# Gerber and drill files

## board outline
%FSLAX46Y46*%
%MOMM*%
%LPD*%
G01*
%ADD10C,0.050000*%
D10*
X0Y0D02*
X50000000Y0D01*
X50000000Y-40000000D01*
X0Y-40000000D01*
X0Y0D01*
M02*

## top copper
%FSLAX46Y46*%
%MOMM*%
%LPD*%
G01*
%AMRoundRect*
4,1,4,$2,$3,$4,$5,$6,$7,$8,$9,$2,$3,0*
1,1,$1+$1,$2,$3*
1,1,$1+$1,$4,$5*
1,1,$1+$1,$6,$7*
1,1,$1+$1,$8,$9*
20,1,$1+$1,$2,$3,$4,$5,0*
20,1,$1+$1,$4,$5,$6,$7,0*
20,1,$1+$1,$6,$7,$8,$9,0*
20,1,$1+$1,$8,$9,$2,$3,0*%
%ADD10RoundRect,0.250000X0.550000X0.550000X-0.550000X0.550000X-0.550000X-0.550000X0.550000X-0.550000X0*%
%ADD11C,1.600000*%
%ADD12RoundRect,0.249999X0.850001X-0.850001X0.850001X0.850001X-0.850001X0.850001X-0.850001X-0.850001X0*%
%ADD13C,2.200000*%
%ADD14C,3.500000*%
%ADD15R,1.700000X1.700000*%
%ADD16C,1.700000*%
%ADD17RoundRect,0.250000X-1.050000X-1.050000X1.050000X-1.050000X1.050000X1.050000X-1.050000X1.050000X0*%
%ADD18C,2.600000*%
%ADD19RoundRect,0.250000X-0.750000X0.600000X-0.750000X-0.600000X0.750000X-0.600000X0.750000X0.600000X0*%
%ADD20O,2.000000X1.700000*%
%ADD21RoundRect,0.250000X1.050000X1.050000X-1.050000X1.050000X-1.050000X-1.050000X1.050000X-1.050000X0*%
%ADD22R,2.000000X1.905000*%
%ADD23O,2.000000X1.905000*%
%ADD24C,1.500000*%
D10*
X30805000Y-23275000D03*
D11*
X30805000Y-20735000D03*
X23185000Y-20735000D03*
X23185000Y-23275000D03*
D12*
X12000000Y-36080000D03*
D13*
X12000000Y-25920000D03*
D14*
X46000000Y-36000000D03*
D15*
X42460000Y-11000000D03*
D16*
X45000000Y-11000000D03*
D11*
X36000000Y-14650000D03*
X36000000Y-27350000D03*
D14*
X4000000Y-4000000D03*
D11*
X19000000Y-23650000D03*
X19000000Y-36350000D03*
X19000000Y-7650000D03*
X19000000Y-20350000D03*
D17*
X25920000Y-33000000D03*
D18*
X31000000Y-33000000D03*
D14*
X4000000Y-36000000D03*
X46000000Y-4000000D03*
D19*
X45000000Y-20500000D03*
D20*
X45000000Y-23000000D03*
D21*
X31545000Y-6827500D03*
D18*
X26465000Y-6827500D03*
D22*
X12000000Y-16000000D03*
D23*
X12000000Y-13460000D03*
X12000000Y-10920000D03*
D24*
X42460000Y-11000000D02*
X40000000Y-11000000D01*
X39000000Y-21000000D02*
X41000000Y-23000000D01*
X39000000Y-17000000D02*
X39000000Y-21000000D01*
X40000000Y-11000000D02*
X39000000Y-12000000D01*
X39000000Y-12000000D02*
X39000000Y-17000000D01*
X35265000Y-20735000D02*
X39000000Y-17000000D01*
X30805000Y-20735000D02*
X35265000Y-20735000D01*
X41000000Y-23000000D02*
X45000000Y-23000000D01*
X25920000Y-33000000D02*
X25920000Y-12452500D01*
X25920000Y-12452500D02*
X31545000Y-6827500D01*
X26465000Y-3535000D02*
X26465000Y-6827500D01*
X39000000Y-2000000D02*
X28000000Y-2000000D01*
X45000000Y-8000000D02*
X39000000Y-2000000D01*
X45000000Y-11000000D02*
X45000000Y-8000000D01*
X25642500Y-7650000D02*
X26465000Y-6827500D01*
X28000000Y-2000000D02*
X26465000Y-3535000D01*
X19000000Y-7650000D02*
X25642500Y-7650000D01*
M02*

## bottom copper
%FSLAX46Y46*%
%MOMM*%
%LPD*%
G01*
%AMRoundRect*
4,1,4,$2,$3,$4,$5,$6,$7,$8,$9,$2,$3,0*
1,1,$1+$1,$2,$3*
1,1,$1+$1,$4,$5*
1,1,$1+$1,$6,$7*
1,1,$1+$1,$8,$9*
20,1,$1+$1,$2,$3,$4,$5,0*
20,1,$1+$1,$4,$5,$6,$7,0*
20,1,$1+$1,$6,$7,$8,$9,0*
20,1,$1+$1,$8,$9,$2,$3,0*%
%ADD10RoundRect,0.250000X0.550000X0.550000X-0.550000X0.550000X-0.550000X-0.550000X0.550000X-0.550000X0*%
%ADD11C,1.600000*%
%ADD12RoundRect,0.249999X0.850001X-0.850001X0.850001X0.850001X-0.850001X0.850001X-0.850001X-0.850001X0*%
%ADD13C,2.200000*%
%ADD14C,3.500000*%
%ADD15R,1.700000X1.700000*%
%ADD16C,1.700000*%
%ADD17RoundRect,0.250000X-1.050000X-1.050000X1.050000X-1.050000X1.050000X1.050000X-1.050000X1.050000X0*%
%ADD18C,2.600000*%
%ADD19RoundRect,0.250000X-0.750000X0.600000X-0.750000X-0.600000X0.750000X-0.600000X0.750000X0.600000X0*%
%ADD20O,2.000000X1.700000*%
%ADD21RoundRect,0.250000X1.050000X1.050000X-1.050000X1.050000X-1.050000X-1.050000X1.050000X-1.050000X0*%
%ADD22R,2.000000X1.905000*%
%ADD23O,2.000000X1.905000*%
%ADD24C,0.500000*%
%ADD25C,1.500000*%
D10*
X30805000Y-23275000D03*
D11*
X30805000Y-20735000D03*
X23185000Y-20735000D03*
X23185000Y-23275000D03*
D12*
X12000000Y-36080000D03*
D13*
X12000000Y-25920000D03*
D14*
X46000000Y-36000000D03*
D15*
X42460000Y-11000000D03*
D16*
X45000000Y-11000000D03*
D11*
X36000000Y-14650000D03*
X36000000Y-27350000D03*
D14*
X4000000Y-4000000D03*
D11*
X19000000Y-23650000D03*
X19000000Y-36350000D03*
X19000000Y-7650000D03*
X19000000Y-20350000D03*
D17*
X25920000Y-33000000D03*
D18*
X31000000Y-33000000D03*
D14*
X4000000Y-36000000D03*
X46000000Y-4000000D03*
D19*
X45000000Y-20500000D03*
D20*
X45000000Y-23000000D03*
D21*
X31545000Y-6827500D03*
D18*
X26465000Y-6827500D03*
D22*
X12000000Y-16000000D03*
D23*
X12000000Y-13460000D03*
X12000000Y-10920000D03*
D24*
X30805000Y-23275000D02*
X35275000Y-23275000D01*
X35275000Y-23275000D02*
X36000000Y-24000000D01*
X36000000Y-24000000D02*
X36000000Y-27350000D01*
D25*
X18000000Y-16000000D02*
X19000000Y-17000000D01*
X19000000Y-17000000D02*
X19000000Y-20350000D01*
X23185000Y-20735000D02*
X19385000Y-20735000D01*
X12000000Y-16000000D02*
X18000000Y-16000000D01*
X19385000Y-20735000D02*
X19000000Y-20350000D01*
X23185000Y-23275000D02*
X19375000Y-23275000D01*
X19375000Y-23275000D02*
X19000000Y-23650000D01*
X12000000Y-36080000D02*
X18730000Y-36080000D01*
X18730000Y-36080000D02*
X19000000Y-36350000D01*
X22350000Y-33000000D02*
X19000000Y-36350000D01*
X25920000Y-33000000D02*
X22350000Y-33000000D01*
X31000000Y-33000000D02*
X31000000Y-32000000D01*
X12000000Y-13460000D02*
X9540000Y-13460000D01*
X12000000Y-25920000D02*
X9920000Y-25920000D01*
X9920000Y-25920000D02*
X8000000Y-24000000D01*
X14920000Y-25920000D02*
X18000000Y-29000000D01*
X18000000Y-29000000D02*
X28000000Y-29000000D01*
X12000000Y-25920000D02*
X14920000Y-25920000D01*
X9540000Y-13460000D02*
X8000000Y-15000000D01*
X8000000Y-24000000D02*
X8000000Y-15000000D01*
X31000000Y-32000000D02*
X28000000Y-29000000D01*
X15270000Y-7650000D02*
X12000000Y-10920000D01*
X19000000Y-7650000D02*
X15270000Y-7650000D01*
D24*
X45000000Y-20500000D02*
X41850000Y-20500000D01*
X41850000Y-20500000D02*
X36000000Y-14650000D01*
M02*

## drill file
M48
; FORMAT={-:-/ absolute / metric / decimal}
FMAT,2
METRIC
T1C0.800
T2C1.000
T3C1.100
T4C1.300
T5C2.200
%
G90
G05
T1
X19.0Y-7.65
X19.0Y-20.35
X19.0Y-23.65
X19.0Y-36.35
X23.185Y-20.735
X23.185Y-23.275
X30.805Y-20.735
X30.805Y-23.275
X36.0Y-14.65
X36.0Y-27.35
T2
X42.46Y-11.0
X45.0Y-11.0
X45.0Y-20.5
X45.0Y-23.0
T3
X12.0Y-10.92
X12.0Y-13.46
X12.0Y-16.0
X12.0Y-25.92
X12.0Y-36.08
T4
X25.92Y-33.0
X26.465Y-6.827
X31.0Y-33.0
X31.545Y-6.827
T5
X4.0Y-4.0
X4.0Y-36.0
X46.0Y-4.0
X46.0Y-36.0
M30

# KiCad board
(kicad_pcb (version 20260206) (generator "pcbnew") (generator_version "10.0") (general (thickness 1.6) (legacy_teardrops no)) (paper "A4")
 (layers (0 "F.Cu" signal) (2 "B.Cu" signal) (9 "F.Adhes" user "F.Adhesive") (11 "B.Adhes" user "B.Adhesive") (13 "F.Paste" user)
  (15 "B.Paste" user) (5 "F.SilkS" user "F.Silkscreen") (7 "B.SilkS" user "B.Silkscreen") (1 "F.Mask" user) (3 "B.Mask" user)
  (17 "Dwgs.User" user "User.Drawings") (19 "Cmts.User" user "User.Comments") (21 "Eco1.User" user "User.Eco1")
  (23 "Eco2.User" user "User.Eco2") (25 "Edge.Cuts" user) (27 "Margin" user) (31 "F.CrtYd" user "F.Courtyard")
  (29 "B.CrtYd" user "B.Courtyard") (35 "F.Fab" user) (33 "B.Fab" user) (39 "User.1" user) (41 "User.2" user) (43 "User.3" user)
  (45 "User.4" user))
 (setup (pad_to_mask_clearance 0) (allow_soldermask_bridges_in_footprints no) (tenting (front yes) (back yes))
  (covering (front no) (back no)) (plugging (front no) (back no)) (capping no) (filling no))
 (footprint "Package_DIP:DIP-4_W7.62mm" (layer "F.Cu") (at 30.805 23.275 180)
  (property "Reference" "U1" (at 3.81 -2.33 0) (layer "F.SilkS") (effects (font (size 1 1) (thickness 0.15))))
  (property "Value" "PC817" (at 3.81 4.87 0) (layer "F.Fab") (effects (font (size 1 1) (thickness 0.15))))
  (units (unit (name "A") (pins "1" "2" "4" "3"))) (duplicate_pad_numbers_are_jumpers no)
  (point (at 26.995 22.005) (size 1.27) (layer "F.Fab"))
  (pad "1" thru_hole roundrect (at 0 0 180) (size 1.6 1.6) (drill 0.8) (layers "*.Cu" "*.Mask") (remove_unused_layers no)
   (roundrect_rratio 0.15625) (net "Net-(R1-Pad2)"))
  (pad "2" thru_hole circle (at 0 2.54 180) (size 1.6 1.6) (drill 0.8) (layers "*.Cu" "*.Mask") (remove_unused_layers no) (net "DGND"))
  (pad "3" thru_hole circle (at 7.62 2.54 180) (size 1.6 1.6) (drill 0.8) (layers "*.Cu" "*.Mask") (remove_unused_layers no)
   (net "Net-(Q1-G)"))
  (pad "4" thru_hole circle (at 7.62 0 180) (size 1.6 1.6) (drill 0.8) (layers "*.Cu" "*.Mask") (remove_unused_layers no)
   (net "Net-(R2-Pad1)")))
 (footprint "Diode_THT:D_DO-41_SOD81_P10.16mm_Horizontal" (layer "F.Cu") (at 12 36.08 90)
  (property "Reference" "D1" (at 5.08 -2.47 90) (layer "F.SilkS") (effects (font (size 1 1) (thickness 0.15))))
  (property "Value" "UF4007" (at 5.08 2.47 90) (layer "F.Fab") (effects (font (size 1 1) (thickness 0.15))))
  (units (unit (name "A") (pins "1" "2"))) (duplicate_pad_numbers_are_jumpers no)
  (pad "1" thru_hole roundrect (at 0 0 90) (size 2.2 2.2) (drill 1.1) (layers "*.Cu" "*.Mask") (remove_unused_layers no)
   (roundrect_rratio 0.113636) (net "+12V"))
  (pad "2" thru_hole circle (at 10.16 0 90) (size 2.2 2.2) (drill 1.1) (layers "*.Cu" "*.Mask") (remove_unused_layers no) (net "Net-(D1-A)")))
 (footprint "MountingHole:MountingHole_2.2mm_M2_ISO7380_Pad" (layer "F.Cu") (at 46 36)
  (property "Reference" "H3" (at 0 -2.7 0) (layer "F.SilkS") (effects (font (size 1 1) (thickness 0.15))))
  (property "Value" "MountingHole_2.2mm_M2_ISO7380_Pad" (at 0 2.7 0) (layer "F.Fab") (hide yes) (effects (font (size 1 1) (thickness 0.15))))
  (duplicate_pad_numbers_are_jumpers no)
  (pad "3" thru_hole circle (at 0 0) (size 3.5 3.5) (drill 2.2) (layers "*.Cu" "*.Mask") (remove_unused_layers no) (zone_connect 2)))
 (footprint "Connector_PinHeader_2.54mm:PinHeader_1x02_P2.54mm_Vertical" (layer "F.Cu") (at 42.46 11 90)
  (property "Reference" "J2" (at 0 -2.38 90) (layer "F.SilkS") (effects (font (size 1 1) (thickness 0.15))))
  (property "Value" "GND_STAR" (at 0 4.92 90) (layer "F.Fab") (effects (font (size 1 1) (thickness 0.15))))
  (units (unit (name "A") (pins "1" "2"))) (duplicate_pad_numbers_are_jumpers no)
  (pad "1" thru_hole rect (at 0 0 90) (size 1.7 1.7) (drill 1) (layers "*.Cu" "*.Mask") (remove_unused_layers no) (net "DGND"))
  (pad "2" thru_hole circle (at 0 2.54 90) (size 1.7 1.7) (drill 1) (layers "*.Cu" "*.Mask") (remove_unused_layers no) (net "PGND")))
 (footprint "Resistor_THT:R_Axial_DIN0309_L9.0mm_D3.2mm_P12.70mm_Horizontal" (layer "F.Cu") (at 36 14.65 -90)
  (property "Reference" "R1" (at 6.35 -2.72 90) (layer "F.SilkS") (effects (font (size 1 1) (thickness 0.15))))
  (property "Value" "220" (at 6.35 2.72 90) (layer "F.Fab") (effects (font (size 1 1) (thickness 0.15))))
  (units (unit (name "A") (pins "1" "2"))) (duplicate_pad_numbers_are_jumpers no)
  (pad "1" thru_hole circle (at 0 0 270) (size 1.6 1.6) (drill 0.8) (layers "*.Cu" "*.Mask") (remove_unused_layers no) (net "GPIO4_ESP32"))
  (pad "2" thru_hole circle (at 12.7 0 270) (size 1.6 1.6) (drill 0.8) (layers "*.Cu" "*.Mask") (remove_unused_layers no)
   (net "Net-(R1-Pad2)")))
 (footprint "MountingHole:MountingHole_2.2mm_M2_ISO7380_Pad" (layer "F.Cu") (at 4 4)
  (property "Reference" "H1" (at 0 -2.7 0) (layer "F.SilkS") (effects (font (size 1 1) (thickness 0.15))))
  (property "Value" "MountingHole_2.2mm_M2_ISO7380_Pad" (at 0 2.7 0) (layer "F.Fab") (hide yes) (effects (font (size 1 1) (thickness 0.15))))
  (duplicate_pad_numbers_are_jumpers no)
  (pad "1" thru_hole circle (at 0 0) (size 3.5 3.5) (drill 2.2) (layers "*.Cu" "*.Mask") (remove_unused_layers no) (zone_connect 2)))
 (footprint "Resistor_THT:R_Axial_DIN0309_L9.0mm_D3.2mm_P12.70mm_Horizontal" (layer "F.Cu") (at 19 23.65 -90)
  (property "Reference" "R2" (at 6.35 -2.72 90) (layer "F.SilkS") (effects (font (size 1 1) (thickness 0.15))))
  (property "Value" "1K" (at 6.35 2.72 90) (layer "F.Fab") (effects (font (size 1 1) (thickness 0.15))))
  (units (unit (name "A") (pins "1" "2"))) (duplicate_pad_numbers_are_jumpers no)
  (pad "1" thru_hole circle (at 0 0 270) (size 1.6 1.6) (drill 0.8) (layers "*.Cu" "*.Mask") (remove_unused_layers no) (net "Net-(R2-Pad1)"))
  (pad "2" thru_hole circle (at 12.7 0 270) (size 1.6 1.6) (drill 0.8) (layers "*.Cu" "*.Mask") (remove_unused_layers no) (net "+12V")))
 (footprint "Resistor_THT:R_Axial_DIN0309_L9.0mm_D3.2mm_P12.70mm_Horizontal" (layer "F.Cu") (at 19 7.65 -90)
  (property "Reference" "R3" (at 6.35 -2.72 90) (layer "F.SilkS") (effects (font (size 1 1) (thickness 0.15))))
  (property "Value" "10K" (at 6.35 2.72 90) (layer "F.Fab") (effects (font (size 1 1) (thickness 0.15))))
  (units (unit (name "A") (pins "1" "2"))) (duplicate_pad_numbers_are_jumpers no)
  (pad "1" thru_hole circle (at 0 0 270) (size 1.6 1.6) (drill 0.8) (layers "*.Cu" "*.Mask") (remove_unused_layers no) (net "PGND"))
  (pad "2" thru_hole circle (at 12.7 0 270) (size 1.6 1.6) (drill 0.8) (layers "*.Cu" "*.Mask") (remove_unused_layers no) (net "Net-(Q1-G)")))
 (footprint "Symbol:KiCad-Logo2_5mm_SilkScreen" (layer "F.Cu") (at 40 33 90)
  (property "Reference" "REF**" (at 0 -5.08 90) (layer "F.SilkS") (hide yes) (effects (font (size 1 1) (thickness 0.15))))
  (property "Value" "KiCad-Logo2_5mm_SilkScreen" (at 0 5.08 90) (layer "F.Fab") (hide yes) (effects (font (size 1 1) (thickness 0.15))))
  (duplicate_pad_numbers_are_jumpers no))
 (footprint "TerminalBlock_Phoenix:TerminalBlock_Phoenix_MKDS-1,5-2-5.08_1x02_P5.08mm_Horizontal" (layer "F.Cu") (at 25.92 33)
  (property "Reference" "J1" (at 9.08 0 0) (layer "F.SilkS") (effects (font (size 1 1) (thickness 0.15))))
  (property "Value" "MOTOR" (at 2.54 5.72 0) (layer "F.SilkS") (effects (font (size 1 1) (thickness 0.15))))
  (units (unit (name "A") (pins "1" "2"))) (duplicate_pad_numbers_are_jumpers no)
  (pad "1" thru_hole roundrect (at 0 0) (size 2.6 2.6) (drill 1.3) (layers "*.Cu" "*.Mask") (remove_unused_layers no)
   (roundrect_rratio 0.096154) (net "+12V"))
  (pad "2" thru_hole circle (at 5.08 0) (size 2.6 2.6) (drill 1.3) (layers "*.Cu" "*.Mask") (remove_unused_layers no) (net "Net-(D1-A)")))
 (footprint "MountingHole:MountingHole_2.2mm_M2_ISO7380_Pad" (layer "F.Cu") (at 4 36)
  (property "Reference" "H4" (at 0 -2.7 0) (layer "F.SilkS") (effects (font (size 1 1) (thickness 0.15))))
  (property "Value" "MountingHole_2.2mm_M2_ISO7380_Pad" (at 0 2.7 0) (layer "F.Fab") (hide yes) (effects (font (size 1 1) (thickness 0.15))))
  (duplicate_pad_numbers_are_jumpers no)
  (pad "4" thru_hole circle (at 0 0) (size 3.5 3.5) (drill 2.2) (layers "*.Cu" "*.Mask") (remove_unused_layers no) (zone_connect 2)))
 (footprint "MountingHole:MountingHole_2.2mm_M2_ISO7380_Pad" (layer "F.Cu") (at 46 4)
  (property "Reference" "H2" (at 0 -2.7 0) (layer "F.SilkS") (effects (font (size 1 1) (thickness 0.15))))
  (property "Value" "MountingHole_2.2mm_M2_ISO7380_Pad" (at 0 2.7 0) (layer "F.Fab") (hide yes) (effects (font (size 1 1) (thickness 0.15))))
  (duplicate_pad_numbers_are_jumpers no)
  (pad "2" thru_hole circle (at 0 0) (size 3.5 3.5) (drill 2.2) (layers "*.Cu" "*.Mask") (remove_unused_layers no) (zone_connect 2)))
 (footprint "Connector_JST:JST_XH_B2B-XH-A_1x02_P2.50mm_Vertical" (layer "F.Cu") (at 45 20.5 -90)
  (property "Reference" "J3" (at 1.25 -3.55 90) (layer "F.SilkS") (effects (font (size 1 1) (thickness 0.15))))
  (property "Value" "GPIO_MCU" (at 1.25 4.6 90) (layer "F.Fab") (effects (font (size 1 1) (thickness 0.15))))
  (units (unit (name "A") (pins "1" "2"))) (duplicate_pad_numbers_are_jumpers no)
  (pad "1" thru_hole roundrect (at 0 0 270) (size 1.7 2) (drill 1) (layers "*.Cu" "*.Mask") (remove_unused_layers no)
   (roundrect_rratio 0.147059) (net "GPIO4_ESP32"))
  (pad "2" thru_hole oval (at 2.5 0 270) (size 1.7 2) (drill 1) (layers "*.Cu" "*.Mask") (remove_unused_layers no) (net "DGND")))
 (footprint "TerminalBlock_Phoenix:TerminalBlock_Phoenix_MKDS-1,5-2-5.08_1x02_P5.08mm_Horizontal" (layer "F.Cu") (at 31.545 6.8275 180)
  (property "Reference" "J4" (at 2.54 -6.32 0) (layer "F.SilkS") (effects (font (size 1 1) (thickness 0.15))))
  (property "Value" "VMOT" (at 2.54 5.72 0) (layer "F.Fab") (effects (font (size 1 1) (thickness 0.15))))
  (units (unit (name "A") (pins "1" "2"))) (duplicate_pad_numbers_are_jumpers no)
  (pad "1" thru_hole roundrect (at 0 0 180) (size 2.6 2.6) (drill 1.3) (layers "*.Cu" "*.Mask") (remove_unused_layers no)
   (roundrect_rratio 0.096154) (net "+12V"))
  (pad "2" thru_hole circle (at 5.08 0 180) (size 2.6 2.6) (drill 1.3) (layers "*.Cu" "*.Mask") (remove_unused_layers no) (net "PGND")))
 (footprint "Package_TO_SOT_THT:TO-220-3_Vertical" (layer "F.Cu") (at 12 16 90)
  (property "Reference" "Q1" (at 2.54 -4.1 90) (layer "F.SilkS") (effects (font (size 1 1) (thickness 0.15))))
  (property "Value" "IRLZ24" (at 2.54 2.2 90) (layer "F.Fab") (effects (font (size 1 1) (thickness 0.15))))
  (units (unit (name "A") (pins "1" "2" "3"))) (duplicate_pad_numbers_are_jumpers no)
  (pad "1" thru_hole rect (at 0 0 90) (size 1.905 2) (drill 1.1) (layers "*.Cu" "*.Mask") (remove_unused_layers no) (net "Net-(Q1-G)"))
  (pad "2" thru_hole oval (at 2.54 0 90) (size 1.905 2) (drill 1.1) (layers "*.Cu" "*.Mask") (remove_unused_layers no) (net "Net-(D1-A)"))
  (pad "3" thru_hole oval (at 5.08 0 90) (size 1.905 2) (drill 1.1) (layers "*.Cu" "*.Mask") (remove_unused_layers no) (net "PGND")))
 (gr_rect (start 0 0) (end 50 40) (stroke (width 0.05) (type default)) (fill no) (layer "Edge.Cuts"))
 (segment (start 30.805 23.275) (end 35.275 23.275) (width 0.5) (layer "B.Cu") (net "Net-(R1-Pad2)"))
 (segment (start 35.275 23.275) (end 36 24) (width 0.5) (layer "B.Cu") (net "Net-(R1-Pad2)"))
 (segment (start 36 24) (end 36 27.35) (width 0.5) (layer "B.Cu") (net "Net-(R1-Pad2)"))
 (segment (start 42.46 11) (end 40 11) (width 1.5) (layer "F.Cu") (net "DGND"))
 (segment (start 39 21) (end 41 23) (width 1.5) (layer "F.Cu") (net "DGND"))
 (segment (start 39 17) (end 39 21) (width 1.5) (layer "F.Cu") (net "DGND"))
 (segment (start 40 11) (end 39 12) (width 1.5) (layer "F.Cu") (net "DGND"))
 (segment (start 39 12) (end 39 17) (width 1.5) (layer "F.Cu") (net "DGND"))
 (segment (start 35.265 20.735) (end 39 17) (width 1.5) (layer "F.Cu") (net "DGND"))
 (segment (start 30.805 20.735) (end 35.265 20.735) (width 1.5) (layer "F.Cu") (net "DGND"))
 (segment (start 41 23) (end 45 23) (width 1.5) (layer "F.Cu") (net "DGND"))
 (segment (start 18 16) (end 19 17) (width 1.5) (layer "B.Cu") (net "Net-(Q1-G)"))
 (segment (start 19 17) (end 19 20.35) (width 1.5) (layer "B.Cu") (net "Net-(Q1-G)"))
 (segment (start 23.185 20.735) (end 19.385 20.735) (width 1.5) (layer "B.Cu") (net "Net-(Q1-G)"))
 (segment (start 12 16) (end 18 16) (width 1.5) (layer "B.Cu") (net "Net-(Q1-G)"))
 (segment (start 19.385 20.735) (end 19 20.35) (width 1.5) (layer "B.Cu") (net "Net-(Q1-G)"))
 (segment (start 23.185 23.275) (end 19.375 23.275) (width 1.5) (layer "B.Cu") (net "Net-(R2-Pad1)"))
 (segment (start 19.375 23.275) (end 19 23.65) (width 1.5) (layer "B.Cu") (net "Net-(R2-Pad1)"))
 (segment (start 25.92 33) (end 25.92 12.4525) (width 1.5) (layer "F.Cu") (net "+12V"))
 (segment (start 25.92 12.4525) (end 31.545 6.8275) (width 1.5) (layer "F.Cu") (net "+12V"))
 (segment (start 12 36.08) (end 18.73 36.08) (width 1.5) (layer "B.Cu") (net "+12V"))
 (segment (start 18.73 36.08) (end 19 36.35) (width 1.5) (layer "B.Cu") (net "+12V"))
 (segment (start 22.35 33) (end 19 36.35) (width 1.5) (layer "B.Cu") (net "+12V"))
 (segment (start 25.92 33) (end 22.35 33) (width 1.5) (layer "B.Cu") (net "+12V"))
 (segment (start 31 33) (end 31 32) (width 1.5) (layer "B.Cu") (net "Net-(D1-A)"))
 (segment (start 12 13.46) (end 9.54 13.46) (width 1.5) (layer "B.Cu") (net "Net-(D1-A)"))
 (segment (start 12 25.92) (end 9.92 25.92) (width 1.5) (layer "B.Cu") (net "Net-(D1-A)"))
 (segment (start 9.92 25.92) (end 8 24) (width 1.5) (layer "B.Cu") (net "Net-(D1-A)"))
 (segment (start 14.92 25.92) (end 18 29) (width 1.5) (layer "B.Cu") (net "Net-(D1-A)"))
 (segment (start 18 29) (end 28 29) (width 1.5) (layer "B.Cu") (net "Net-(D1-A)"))
 (segment (start 12 25.92) (end 14.92 25.92) (width 1.5) (layer "B.Cu") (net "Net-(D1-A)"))
 (segment (start 9.54 13.46) (end 8 15) (width 1.5) (layer "B.Cu") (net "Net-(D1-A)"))
 (segment (start 8 24) (end 8 15) (width 1.5) (layer "B.Cu") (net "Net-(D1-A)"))
 (segment (start 31 32) (end 28 29) (width 1.5) (layer "B.Cu") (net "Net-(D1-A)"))
 (segment (start 26.465 3.535) (end 26.465 6.8275) (width 1.5) (layer "F.Cu") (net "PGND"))
 (segment (start 39 2) (end 28 2) (width 1.5) (layer "F.Cu") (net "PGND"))
 (segment (start 45 8) (end 39 2) (width 1.5) (layer "F.Cu") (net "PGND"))
 (segment (start 45 11) (end 45 8) (width 1.5) (layer "F.Cu") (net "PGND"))
 (segment (start 25.6425 7.65) (end 26.465 6.8275) (width 1.5) (layer "F.Cu") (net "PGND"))
 (segment (start 28 2) (end 26.465 3.535) (width 1.5) (layer "F.Cu") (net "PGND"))
 (segment (start 19 7.65) (end 25.6425 7.65) (width 1.5) (layer "F.Cu") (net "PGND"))
 (segment (start 15.27 7.65) (end 12 10.92) (width 1.5) (layer "B.Cu") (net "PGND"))
 (segment (start 19 7.65) (end 15.27 7.65) (width 1.5) (layer "B.Cu") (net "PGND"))
 (segment (start 45 20.5) (end 41.85 20.5) (width 0.5) (layer "B.Cu") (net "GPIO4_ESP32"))
 (segment (start 41.85 20.5) (end 36 14.65) (width 0.5) (layer "B.Cu") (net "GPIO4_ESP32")))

